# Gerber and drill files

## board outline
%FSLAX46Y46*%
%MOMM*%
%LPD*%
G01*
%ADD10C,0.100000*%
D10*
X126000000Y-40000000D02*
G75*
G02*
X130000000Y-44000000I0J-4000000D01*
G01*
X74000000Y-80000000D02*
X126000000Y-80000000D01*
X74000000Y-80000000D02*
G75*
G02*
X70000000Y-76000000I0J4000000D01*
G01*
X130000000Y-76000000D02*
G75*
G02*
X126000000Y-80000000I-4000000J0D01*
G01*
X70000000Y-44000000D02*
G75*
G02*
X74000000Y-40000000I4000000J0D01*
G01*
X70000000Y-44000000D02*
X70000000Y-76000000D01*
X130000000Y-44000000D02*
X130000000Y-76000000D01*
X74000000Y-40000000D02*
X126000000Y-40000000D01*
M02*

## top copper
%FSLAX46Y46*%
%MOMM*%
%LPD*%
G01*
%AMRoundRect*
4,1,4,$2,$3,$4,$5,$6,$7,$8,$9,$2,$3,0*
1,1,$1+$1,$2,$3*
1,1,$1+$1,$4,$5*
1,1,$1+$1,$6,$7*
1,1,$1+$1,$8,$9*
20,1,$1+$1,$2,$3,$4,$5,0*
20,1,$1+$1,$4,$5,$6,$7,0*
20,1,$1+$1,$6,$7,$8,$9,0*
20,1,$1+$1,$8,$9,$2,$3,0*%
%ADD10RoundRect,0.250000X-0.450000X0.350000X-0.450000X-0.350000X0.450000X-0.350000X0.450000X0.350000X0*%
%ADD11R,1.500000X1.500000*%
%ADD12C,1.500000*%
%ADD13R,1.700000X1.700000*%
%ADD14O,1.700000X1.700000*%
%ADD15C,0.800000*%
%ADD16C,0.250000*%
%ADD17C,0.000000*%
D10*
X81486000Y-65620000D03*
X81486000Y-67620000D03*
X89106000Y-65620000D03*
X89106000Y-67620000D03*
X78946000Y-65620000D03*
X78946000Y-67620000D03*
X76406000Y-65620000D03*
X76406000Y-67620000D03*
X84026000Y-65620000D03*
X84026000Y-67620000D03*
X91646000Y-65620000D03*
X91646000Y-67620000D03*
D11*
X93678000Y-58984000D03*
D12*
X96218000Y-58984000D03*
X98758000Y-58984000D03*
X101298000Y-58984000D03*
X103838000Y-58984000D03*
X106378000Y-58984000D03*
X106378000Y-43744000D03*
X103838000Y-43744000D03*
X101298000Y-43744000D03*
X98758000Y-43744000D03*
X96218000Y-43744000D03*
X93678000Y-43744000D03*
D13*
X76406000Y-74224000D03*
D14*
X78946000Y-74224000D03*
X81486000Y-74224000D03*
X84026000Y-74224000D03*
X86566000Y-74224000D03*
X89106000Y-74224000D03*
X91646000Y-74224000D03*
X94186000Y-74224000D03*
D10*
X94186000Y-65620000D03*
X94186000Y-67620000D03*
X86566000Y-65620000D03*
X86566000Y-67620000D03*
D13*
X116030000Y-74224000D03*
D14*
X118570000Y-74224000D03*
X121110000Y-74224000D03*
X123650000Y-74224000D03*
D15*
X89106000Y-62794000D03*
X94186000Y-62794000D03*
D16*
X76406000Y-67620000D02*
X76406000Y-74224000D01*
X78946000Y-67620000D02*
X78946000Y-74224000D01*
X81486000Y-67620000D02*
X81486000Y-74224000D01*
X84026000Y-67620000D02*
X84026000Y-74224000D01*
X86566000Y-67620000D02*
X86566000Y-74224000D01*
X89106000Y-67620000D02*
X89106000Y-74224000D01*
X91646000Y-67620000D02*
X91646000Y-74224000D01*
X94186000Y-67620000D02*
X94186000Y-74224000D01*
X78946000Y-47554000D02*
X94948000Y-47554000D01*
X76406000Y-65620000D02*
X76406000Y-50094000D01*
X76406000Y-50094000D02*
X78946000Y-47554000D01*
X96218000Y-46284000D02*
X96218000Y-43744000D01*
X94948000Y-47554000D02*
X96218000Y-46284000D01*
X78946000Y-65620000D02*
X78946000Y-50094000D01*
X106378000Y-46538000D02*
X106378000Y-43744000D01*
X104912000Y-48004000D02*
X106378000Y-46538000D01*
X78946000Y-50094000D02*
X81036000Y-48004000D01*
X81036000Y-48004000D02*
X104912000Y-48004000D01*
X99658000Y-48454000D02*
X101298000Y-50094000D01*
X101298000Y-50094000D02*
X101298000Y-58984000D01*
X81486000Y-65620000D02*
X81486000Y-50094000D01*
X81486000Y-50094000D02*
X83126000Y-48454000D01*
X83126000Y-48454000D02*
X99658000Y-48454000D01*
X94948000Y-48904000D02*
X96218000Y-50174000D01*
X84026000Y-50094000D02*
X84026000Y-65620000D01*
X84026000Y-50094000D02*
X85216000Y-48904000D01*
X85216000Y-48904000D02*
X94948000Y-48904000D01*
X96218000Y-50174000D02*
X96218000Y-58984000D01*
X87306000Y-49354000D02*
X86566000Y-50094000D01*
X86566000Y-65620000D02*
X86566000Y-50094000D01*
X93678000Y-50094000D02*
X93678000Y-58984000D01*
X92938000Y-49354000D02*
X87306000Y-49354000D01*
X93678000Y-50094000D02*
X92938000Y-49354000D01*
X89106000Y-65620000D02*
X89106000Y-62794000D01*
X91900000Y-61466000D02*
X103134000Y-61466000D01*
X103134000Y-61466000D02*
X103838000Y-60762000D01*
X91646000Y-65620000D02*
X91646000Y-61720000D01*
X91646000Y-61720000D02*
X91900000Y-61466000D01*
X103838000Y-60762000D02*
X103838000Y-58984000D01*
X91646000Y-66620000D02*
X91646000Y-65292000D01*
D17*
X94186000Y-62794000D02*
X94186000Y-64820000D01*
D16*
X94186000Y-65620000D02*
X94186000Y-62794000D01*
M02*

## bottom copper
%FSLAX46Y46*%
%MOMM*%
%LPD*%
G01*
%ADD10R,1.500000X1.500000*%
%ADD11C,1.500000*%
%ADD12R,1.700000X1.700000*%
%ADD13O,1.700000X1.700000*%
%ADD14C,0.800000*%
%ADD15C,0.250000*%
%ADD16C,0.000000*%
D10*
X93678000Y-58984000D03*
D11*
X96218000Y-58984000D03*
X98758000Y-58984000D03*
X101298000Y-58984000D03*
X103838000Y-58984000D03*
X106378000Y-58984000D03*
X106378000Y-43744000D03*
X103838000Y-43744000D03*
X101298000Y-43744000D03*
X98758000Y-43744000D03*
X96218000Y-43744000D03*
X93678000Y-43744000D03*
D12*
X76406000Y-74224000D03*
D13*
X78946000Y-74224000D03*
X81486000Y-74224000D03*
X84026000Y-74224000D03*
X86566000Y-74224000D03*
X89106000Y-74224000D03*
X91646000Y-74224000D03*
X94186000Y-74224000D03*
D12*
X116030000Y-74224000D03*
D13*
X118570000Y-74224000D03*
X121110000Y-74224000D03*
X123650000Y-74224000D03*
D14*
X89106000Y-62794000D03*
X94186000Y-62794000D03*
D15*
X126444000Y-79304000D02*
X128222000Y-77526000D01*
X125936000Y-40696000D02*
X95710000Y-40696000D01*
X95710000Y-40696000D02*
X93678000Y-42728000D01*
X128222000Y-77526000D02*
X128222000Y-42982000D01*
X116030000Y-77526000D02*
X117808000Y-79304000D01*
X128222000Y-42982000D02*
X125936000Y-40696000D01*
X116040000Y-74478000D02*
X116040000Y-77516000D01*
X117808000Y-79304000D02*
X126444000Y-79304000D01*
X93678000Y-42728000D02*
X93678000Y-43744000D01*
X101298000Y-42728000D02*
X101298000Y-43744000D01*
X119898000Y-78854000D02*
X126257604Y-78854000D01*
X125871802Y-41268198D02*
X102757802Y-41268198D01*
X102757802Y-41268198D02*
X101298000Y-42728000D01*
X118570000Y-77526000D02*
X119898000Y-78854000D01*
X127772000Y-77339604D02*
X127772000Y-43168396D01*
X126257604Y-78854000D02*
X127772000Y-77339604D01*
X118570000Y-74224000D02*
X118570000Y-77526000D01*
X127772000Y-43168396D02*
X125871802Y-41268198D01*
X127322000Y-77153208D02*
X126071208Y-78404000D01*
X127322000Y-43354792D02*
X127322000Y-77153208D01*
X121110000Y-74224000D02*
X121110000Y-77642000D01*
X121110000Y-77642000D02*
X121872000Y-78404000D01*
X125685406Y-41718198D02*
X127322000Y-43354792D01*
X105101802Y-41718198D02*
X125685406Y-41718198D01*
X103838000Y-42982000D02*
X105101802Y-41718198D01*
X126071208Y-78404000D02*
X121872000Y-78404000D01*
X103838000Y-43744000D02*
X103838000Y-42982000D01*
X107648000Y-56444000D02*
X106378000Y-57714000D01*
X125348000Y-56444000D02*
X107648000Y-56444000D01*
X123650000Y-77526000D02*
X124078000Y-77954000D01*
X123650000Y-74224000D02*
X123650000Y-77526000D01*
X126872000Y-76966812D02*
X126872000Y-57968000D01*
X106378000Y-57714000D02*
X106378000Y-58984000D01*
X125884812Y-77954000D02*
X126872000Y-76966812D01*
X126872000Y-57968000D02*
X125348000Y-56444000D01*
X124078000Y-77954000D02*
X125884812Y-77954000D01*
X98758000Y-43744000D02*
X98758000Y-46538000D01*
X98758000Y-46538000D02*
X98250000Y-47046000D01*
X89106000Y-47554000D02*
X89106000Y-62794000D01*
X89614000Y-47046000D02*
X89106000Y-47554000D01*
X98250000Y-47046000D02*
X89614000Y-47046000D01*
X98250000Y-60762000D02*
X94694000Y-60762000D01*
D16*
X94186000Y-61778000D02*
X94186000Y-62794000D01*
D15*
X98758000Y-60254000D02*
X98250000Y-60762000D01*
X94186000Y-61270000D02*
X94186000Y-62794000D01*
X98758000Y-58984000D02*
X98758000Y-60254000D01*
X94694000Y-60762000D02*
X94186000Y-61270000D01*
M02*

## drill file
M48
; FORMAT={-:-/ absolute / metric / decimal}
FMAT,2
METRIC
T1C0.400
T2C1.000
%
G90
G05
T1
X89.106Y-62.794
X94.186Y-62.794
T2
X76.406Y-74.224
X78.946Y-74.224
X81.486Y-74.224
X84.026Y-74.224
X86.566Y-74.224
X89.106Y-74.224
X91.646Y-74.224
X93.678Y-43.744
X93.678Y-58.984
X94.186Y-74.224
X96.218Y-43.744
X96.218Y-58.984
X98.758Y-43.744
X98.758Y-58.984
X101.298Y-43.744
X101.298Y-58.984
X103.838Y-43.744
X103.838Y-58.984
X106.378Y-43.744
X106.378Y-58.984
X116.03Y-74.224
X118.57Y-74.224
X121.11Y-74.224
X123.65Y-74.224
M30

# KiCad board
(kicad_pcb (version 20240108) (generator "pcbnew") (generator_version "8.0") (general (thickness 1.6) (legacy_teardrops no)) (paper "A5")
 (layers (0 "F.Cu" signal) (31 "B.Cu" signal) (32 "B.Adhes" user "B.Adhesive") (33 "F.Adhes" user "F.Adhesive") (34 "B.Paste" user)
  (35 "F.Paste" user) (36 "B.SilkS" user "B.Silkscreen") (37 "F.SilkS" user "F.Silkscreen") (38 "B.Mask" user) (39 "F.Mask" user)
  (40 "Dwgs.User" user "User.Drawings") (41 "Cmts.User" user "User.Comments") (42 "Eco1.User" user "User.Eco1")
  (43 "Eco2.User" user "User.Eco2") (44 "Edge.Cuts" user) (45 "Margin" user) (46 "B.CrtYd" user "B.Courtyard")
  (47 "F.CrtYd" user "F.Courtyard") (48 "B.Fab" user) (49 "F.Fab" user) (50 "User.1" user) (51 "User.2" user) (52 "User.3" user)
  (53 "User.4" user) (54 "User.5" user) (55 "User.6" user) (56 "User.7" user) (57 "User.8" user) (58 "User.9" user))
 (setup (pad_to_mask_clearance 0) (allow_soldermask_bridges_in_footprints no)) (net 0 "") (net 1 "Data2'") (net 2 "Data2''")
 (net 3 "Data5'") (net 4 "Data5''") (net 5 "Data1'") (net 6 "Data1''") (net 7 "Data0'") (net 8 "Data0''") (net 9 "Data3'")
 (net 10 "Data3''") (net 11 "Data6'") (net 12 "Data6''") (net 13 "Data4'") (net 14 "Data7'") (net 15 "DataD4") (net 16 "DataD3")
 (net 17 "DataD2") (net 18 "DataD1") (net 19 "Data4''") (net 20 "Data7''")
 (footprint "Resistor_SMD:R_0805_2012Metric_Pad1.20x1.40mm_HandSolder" (layer "F.Cu") (at 81.486 66.62 -90)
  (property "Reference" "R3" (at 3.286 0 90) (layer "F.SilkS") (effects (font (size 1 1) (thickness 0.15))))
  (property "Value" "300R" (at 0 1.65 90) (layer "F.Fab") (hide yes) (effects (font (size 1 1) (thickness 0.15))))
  (pad "1" smd roundrect (at -1 0 270) (size 1.2 1.4) (layers "F.Cu" "F.Paste" "F.Mask") (roundrect_rratio 0.2083333333) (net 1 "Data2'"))
  (pad "2" smd roundrect (at 1 0 270) (size 1.2 1.4) (layers "F.Cu" "F.Paste" "F.Mask") (roundrect_rratio 0.2083333333) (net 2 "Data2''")))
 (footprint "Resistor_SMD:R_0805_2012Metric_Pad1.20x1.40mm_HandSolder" (layer "F.Cu") (at 89.106 66.62 -90)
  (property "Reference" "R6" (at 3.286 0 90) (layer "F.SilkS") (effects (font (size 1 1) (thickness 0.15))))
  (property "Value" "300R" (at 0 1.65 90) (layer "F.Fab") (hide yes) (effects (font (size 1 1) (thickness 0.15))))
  (pad "1" smd roundrect (at -1 0 270) (size 1.2 1.4) (layers "F.Cu" "F.Paste" "F.Mask") (roundrect_rratio 0.2083333333) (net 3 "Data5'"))
  (pad "2" smd roundrect (at 1 0 270) (size 1.2 1.4) (layers "F.Cu" "F.Paste" "F.Mask") (roundrect_rratio 0.2083333333) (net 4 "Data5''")))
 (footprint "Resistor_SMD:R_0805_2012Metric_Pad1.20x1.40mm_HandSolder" (layer "F.Cu") (at 78.946 66.62 -90)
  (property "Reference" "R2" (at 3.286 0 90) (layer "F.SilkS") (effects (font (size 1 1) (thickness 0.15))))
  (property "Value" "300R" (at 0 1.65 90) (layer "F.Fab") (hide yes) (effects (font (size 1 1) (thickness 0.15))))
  (pad "1" smd roundrect (at -1 0 270) (size 1.2 1.4) (layers "F.Cu" "F.Paste" "F.Mask") (roundrect_rratio 0.2083333333) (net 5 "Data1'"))
  (pad "2" smd roundrect (at 1 0 270) (size 1.2 1.4) (layers "F.Cu" "F.Paste" "F.Mask") (roundrect_rratio 0.2083333333) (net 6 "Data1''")))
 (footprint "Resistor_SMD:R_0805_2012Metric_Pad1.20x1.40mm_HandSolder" (layer "F.Cu") (at 76.406 66.62 -90)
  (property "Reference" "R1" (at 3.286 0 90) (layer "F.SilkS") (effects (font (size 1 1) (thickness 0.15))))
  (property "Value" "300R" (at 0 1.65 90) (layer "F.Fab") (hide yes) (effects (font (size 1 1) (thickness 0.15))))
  (pad "1" smd roundrect (at -1 0 270) (size 1.2 1.4) (layers "F.Cu" "F.Paste" "F.Mask") (roundrect_rratio 0.2083333333) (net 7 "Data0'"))
  (pad "2" smd roundrect (at 1 0 270) (size 1.2 1.4) (layers "F.Cu" "F.Paste" "F.Mask") (roundrect_rratio 0.2083333333) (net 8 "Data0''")))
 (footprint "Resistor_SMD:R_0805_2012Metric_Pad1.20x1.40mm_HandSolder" (layer "F.Cu") (at 84.026 66.62 -90)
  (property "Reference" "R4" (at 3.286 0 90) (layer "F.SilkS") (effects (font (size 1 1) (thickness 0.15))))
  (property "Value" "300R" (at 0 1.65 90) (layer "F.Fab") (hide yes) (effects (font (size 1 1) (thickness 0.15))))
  (pad "1" smd roundrect (at -1 0 270) (size 1.2 1.4) (layers "F.Cu" "F.Paste" "F.Mask") (roundrect_rratio 0.2083333333) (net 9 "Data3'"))
  (pad "2" smd roundrect (at 1 0 270) (size 1.2 1.4) (layers "F.Cu" "F.Paste" "F.Mask") (roundrect_rratio 0.2083333333) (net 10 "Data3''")))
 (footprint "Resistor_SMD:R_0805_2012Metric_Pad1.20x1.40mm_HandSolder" (layer "F.Cu") (at 91.646 66.62 -90)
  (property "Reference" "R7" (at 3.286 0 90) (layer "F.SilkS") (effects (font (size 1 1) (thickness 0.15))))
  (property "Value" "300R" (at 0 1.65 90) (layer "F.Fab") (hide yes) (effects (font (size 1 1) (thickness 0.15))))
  (pad "1" smd roundrect (at -1 0 270) (size 1.2 1.4) (layers "F.Cu" "F.Paste" "F.Mask") (roundrect_rratio 0.2083333333) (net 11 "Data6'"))
  (pad "2" smd roundrect (at 1 0 270) (size 1.2 1.4) (layers "F.Cu" "F.Paste" "F.Mask") (roundrect_rratio 0.2083333333) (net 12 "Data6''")))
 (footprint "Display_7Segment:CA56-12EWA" (layer "F.Cu") (at 93.678 58.984 90)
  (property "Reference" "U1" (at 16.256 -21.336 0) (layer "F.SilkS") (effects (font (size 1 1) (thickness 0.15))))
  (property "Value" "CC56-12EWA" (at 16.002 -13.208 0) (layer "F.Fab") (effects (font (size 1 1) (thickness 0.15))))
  (pad "1" thru_hole rect (at 0 0 90) (size 1.5 1.5) (drill 1) (layers "*.Cu" "*.Mask") (remove_unused_layers no) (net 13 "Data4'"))
  (pad "2" thru_hole circle (at 0 2.54 90) (size 1.5 1.5) (drill 1) (layers "*.Cu" "*.Mask") (remove_unused_layers no) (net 9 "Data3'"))
  (pad "3" thru_hole circle (at 0 5.08 90) (size 1.5 1.5) (drill 1) (layers "*.Cu" "*.Mask") (remove_unused_layers no) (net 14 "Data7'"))
  (pad "4" thru_hole circle (at 0 7.62 90) (size 1.5 1.5) (drill 1) (layers "*.Cu" "*.Mask") (remove_unused_layers no) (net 1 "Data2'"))
  (pad "5" thru_hole circle (at 0 10.16 90) (size 1.5 1.5) (drill 1) (layers "*.Cu" "*.Mask") (remove_unused_layers no) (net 11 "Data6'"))
  (pad "6" thru_hole circle (at 0 12.7 90) (size 1.5 1.5) (drill 1) (layers "*.Cu" "*.Mask") (remove_unused_layers no) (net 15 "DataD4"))
  (pad "7" thru_hole circle (at 15.24 12.7 90) (size 1.5 1.5) (drill 1) (layers "*.Cu" "*.Mask") (remove_unused_layers no) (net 5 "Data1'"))
  (pad "8" thru_hole circle (at 15.24 10.16 90) (size 1.5 1.5) (drill 1) (layers "*.Cu" "*.Mask") (remove_unused_layers no)
   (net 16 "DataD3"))
  (pad "9" thru_hole circle (at 15.24 7.62 90) (size 1.5 1.5) (drill 1) (layers "*.Cu" "*.Mask") (remove_unused_layers no) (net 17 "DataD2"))
  (pad "10" thru_hole circle (at 15.24 5.08 90) (size 1.5 1.5) (drill 1) (layers "*.Cu" "*.Mask") (remove_unused_layers no) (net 3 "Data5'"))
  (pad "11" thru_hole circle (at 15.24 2.54 90) (size 1.5 1.5) (drill 1) (layers "*.Cu" "*.Mask") (remove_unused_layers no) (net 7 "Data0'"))
  (pad "12" thru_hole circle (at 15.24 0 90) (size 1.5 1.5) (drill 1) (layers "*.Cu" "*.Mask") (remove_unused_layers no) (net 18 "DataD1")))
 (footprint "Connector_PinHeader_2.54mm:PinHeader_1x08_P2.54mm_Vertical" (layer "F.Cu") (at 76.406 74.224 90)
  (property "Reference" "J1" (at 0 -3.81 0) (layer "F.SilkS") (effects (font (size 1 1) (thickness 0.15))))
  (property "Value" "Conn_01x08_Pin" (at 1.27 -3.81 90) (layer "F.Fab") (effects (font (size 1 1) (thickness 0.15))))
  (pad "1" thru_hole rect (at 0 0 90) (size 1.7 1.7) (drill 1) (layers "*.Cu" "*.Mask") (remove_unused_layers no) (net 8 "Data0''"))
  (pad "2" thru_hole oval (at 0 2.54 90) (size 1.7 1.7) (drill 1) (layers "*.Cu" "*.Mask") (remove_unused_layers no) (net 6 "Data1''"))
  (pad "3" thru_hole oval (at 0 5.08 90) (size 1.7 1.7) (drill 1) (layers "*.Cu" "*.Mask") (remove_unused_layers no) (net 2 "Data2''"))
  (pad "4" thru_hole oval (at 0 7.62 90) (size 1.7 1.7) (drill 1) (layers "*.Cu" "*.Mask") (remove_unused_layers no) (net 10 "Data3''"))
  (pad "5" thru_hole oval (at 0 10.16 90) (size 1.7 1.7) (drill 1) (layers "*.Cu" "*.Mask") (remove_unused_layers no) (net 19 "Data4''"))
  (pad "6" thru_hole oval (at 0 12.7 90) (size 1.7 1.7) (drill 1) (layers "*.Cu" "*.Mask") (remove_unused_layers no) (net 4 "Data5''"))
  (pad "7" thru_hole oval (at 0 15.24 90) (size 1.7 1.7) (drill 1) (layers "*.Cu" "*.Mask") (remove_unused_layers no) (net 12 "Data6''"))
  (pad "8" thru_hole oval (at 0 17.78 90) (size 1.7 1.7) (drill 1) (layers "*.Cu" "*.Mask") (remove_unused_layers no) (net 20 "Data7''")))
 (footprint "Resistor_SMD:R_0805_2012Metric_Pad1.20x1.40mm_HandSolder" (layer "F.Cu") (at 94.186 66.62 -90)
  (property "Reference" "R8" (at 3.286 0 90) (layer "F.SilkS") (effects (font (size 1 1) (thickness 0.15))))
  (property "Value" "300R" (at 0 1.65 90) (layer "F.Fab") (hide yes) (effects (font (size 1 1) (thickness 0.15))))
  (pad "1" smd roundrect (at -1 0 270) (size 1.2 1.4) (layers "F.Cu" "F.Paste" "F.Mask") (roundrect_rratio 0.2083333333) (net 14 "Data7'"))
  (pad "2" smd roundrect (at 1 0 270) (size 1.2 1.4) (layers "F.Cu" "F.Paste" "F.Mask") (roundrect_rratio 0.2083333333) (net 20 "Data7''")))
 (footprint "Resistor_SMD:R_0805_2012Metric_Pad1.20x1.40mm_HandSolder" (layer "F.Cu") (at 86.566 66.62 -90)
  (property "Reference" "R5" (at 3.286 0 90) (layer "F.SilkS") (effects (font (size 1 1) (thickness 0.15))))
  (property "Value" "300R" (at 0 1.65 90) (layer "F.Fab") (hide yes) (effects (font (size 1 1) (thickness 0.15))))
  (pad "1" smd roundrect (at -1 0 270) (size 1.2 1.4) (layers "F.Cu" "F.Paste" "F.Mask") (roundrect_rratio 0.2083333333) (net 13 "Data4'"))
  (pad "2" smd roundrect (at 1 0 270) (size 1.2 1.4) (layers "F.Cu" "F.Paste" "F.Mask") (roundrect_rratio 0.2083333333) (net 19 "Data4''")))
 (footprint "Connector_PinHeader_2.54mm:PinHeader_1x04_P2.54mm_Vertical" (layer "F.Cu") (at 116.03 74.224 90)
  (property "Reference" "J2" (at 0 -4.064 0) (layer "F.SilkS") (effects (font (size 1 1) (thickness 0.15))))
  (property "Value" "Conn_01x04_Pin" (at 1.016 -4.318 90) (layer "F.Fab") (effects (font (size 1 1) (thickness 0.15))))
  (pad "1" thru_hole rect (at 0 0 90) (size 1.7 1.7) (drill 1) (layers "*.Cu" "*.Mask") (remove_unused_layers no) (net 18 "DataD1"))
  (pad "2" thru_hole oval (at 0 2.54 90) (size 1.7 1.7) (drill 1) (layers "*.Cu" "*.Mask") (remove_unused_layers no) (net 17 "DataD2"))
  (pad "3" thru_hole oval (at 0 5.08 90) (size 1.7 1.7) (drill 1) (layers "*.Cu" "*.Mask") (remove_unused_layers no) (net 16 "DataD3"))
  (pad "4" thru_hole oval (at 0 7.62 90) (size 1.7 1.7) (drill 1) (layers "*.Cu" "*.Mask") (remove_unused_layers no) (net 15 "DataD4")))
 (gr_arc (start 126 40) (mid 128.828427 41.171573) (end 130 44) (stroke (width 0.1) (type default)) (layer "Edge.Cuts"))
 (gr_line (start 74 80) (end 126 80) (stroke (width 0.1) (type default)) (layer "Edge.Cuts"))
 (gr_arc (start 74 80) (mid 71.171573 78.828427) (end 70 76) (stroke (width 0.1) (type default)) (layer "Edge.Cuts"))
 (gr_arc (start 130 76) (mid 128.828427 78.828427) (end 126 80) (stroke (width 0.1) (type default)) (layer "Edge.Cuts"))
 (gr_arc (start 70 44) (mid 71.171573 41.171573) (end 74 40) (stroke (width 0.1) (type default)) (layer "Edge.Cuts"))
 (gr_line (start 70 44) (end 70 76) (stroke (width 0.1) (type default)) (layer "Edge.Cuts"))
 (gr_line (start 130 44) (end 130 76) (stroke (width 0.1) (type default)) (layer "Edge.Cuts"))
 (gr_line (start 74 40) (end 126 40) (stroke (width 0.1) (type default)) (layer "Edge.Cuts"))
 (segment (start 76.406 67.62) (end 76.406 74.224) (width 0.25) (layer "F.Cu") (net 8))
 (segment (start 78.946 67.62) (end 78.946 74.224) (width 0.25) (layer "F.Cu") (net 6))
 (segment (start 81.486 67.62) (end 81.486 74.224) (width 0.25) (layer "F.Cu") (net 2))
 (segment (start 84.026 67.62) (end 84.026 74.224) (width 0.25) (layer "F.Cu") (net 10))
 (segment (start 86.566 67.62) (end 86.566 74.224) (width 0.25) (layer "F.Cu") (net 19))
 (segment (start 89.106 67.62) (end 89.106 74.224) (width 0.25) (layer "F.Cu") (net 4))
 (segment (start 91.646 67.62) (end 91.646 74.224) (width 0.25) (layer "F.Cu") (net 12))
 (segment (start 94.186 67.62) (end 94.186 74.224) (width 0.25) (layer "F.Cu") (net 20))
 (segment (start 126.444 79.304) (end 128.222 77.526) (width 0.25) (layer "B.Cu") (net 18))
 (segment (start 125.936 40.696) (end 95.71 40.696) (width 0.25) (layer "B.Cu") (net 18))
 (segment (start 95.71 40.696) (end 93.678 42.728) (width 0.25) (layer "B.Cu") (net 18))
 (segment (start 128.222 77.526) (end 128.222 42.982) (width 0.25) (layer "B.Cu") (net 18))
 (segment (start 116.03 77.526) (end 117.808 79.304) (width 0.25) (layer "B.Cu") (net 18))
 (segment (start 128.222 42.982) (end 125.936 40.696) (width 0.25) (layer "B.Cu") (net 18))
 (segment (start 116.04 74.478) (end 116.04 77.516) (width 0.25) (layer "B.Cu") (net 18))
 (segment (start 117.808 79.304) (end 126.444 79.304) (width 0.25) (layer "B.Cu") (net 18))
 (segment (start 93.678 42.728) (end 93.678 43.744) (width 0.25) (layer "B.Cu") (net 18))
 (segment (start 101.298 42.728) (end 101.298 43.744) (width 0.25) (layer "B.Cu") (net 17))
 (segment (start 119.898 78.854) (end 126.257604 78.854) (width 0.25) (layer "B.Cu") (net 17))
 (segment (start 125.871802 41.268198) (end 102.757802 41.268198) (width 0.25) (layer "B.Cu") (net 17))
 (segment (start 102.757802 41.268198) (end 101.298 42.728) (width 0.25) (layer "B.Cu") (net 17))
 (segment (start 118.57 77.526) (end 119.898 78.854) (width 0.25) (layer "B.Cu") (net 17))
 (segment (start 127.772 77.339604) (end 127.772 43.168396) (width 0.25) (layer "B.Cu") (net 17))
 (segment (start 126.257604 78.854) (end 127.772 77.339604) (width 0.25) (layer "B.Cu") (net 17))
 (segment (start 118.57 74.224) (end 118.57 77.526) (width 0.25) (layer "B.Cu") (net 17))
 (segment (start 127.772 43.168396) (end 125.871802 41.268198) (width 0.25) (layer "B.Cu") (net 17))
 (segment (start 127.322 77.153208) (end 126.071208 78.404) (width 0.25) (layer "B.Cu") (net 16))
 (segment (start 127.322 43.354792) (end 127.322 77.153208) (width 0.25) (layer "B.Cu") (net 16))
 (segment (start 121.11 74.224) (end 121.11 77.642) (width 0.25) (layer "B.Cu") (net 16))
 (segment (start 121.11 77.642) (end 121.872 78.404) (width 0.25) (layer "B.Cu") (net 16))
 (segment (start 125.685406 41.718198) (end 127.322 43.354792) (width 0.25) (layer "B.Cu") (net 16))
 (segment (start 105.101802 41.718198) (end 125.685406 41.718198) (width 0.25) (layer "B.Cu") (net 16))
 (segment (start 103.838 42.982) (end 105.101802 41.718198) (width 0.25) (layer "B.Cu") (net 16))
 (segment (start 126.071208 78.404) (end 121.872 78.404) (width 0.25) (layer "B.Cu") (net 16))
 (segment (start 103.838 43.744) (end 103.838 42.982) (width 0.25) (layer "B.Cu") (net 16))
 (segment (start 107.648 56.444) (end 106.378 57.714) (width 0.25) (layer "B.Cu") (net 15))
 (segment (start 125.348 56.444) (end 107.648 56.444) (width 0.25) (layer "B.Cu") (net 15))
 (segment (start 123.65 77.526) (end 124.078 77.954) (width 0.25) (layer "B.Cu") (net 15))
 (segment (start 123.65 74.224) (end 123.65 77.526) (width 0.25) (layer "B.Cu") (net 15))
 (segment (start 126.872 76.966812) (end 126.872 57.968) (width 0.25) (layer "B.Cu") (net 15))
 (segment (start 106.378 57.714) (end 106.378 58.984) (width 0.25) (layer "B.Cu") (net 15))
 (segment (start 125.884812 77.954) (end 126.872 76.966812) (width 0.25) (layer "B.Cu") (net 15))
 (segment (start 126.872 57.968) (end 125.348 56.444) (width 0.25) (layer "B.Cu") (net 15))
 (segment (start 124.078 77.954) (end 125.884812 77.954) (width 0.25) (layer "B.Cu") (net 15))
 (segment (start 78.946 47.554) (end 94.948 47.554) (width 0.25) (layer "F.Cu") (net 7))
 (segment (start 76.406 65.62) (end 76.406 50.094) (width 0.25) (layer "F.Cu") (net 7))
 (segment (start 76.406 50.094) (end 78.946 47.554) (width 0.25) (layer "F.Cu") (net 7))
 (segment (start 96.218 46.284) (end 96.218 43.744) (width 0.25) (layer "F.Cu") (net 7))
 (segment (start 94.948 47.554) (end 96.218 46.284) (width 0.25) (layer "F.Cu") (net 7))
 (segment (start 78.946 65.62) (end 78.946 50.094) (width 0.25) (layer "F.Cu") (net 5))
 (segment (start 106.378 46.538) (end 106.378 43.744) (width 0.25) (layer "F.Cu") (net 5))
 (segment (start 104.912 48.004) (end 106.378 46.538) (width 0.25) (layer "F.Cu") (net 5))
 (segment (start 78.946 50.094) (end 81.036 48.004) (width 0.25) (layer "F.Cu") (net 5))
 (segment (start 81.036 48.004) (end 104.912 48.004) (width 0.25) (layer "F.Cu") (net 5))
 (segment (start 99.658 48.454) (end 101.298 50.094) (width 0.25) (layer "F.Cu") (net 1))
 (segment (start 101.298 50.094) (end 101.298 58.984) (width 0.25) (layer "F.Cu") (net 1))
 (segment (start 81.486 65.62) (end 81.486 50.094) (width 0.25) (layer "F.Cu") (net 1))
 (segment (start 81.486 50.094) (end 83.126 48.454) (width 0.25) (layer "F.Cu") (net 1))
 (segment (start 83.126 48.454) (end 99.658 48.454) (width 0.25) (layer "F.Cu") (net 1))
 (segment (start 94.948 48.904) (end 96.218 50.174) (width 0.25) (layer "F.Cu") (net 9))
 (segment (start 84.026 50.094) (end 84.026 65.62) (width 0.25) (layer "F.Cu") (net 9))
 (segment (start 84.026 50.094) (end 85.216 48.904) (width 0.25) (layer "F.Cu") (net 9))
 (segment (start 85.216 48.904) (end 94.948 48.904) (width 0.25) (layer "F.Cu") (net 9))
 (segment (start 96.218 50.174) (end 96.218 58.984) (width 0.25) (layer "F.Cu") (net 9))
 (segment (start 87.306 49.354) (end 86.566 50.094) (width 0.25) (layer "F.Cu") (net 13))
 (segment (start 86.566 65.62) (end 86.566 50.094) (width 0.25) (layer "F.Cu") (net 13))
 (segment (start 93.678 50.094) (end 93.678 58.984) (width 0.25) (layer "F.Cu") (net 13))
 (segment (start 92.938 49.354) (end 87.306 49.354) (width 0.25) (layer "F.Cu") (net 13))
 (segment (start 93.678 50.094) (end 92.938 49.354) (width 0.25) (layer "F.Cu") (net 13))
 (segment (start 89.106 65.62) (end 89.106 62.794) (width 0.25) (layer "F.Cu") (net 3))
 (via (at 89.106 62.794) (size 0.8) (drill 0.4) (layers "F.Cu" "B.Cu") (free yes) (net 3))
 (segment (start 98.758 43.744) (end 98.758 46.538) (width 0.25) (layer "B.Cu") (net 3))
 (segment (start 98.758 46.538) (end 98.25 47.046) (width 0.25) (layer "B.Cu") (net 3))
 (segment (start 89.106 47.554) (end 89.106 62.794) (width 0.25) (layer "B.Cu") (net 3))
 (segment (start 89.614 47.046) (end 89.106 47.554) (width 0.25) (layer "B.Cu") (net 3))
 (segment (start 98.25 47.046) (end 89.614 47.046) (width 0.25) (layer "B.Cu") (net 3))
 (segment (start 91.9 61.466) (end 103.134 61.466) (width 0.25) (layer "F.Cu") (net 11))
 (segment (start 103.134 61.466) (end 103.838 60.762) (width 0.25) (layer "F.Cu") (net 11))
 (segment (start 91.646 65.62) (end 91.646 61.72) (width 0.25) (layer "F.Cu") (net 11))
 (segment (start 91.646 61.72) (end 91.9 61.466) (width 0.25) (layer "F.Cu") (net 11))
 (segment (start 103.838 60.762) (end 103.838 58.984) (width 0.25) (layer "F.Cu") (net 11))
 (segment (start 91.646 66.62) (end 91.646 65.292) (width 0.25) (layer "F.Cu") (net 11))
 (segment (start 94.186 62.794) (end 94.186 64.82) (width 0) (layer "F.Cu") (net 14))
 (segment (start 94.186 65.62) (end 94.186 62.794) (width 0.25) (layer "F.Cu") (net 14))
 (via (at 94.186 62.794) (size 0.8) (drill 0.4) (layers "F.Cu" "B.Cu") (free yes) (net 14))
 (segment (start 98.25 60.762) (end 94.694 60.762) (width 0.25) (layer "B.Cu") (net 14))
 (segment (start 94.186 61.778) (end 94.186 62.794) (width 0) (layer "B.Cu") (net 14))
 (segment (start 98.758 60.254) (end 98.25 60.762) (width 0.25) (layer "B.Cu") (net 14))
 (segment (start 94.186 61.27) (end 94.186 62.794) (width 0.25) (layer "B.Cu") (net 14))
 (segment (start 98.758 58.984) (end 98.758 60.254) (width 0.25) (layer "B.Cu") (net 14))
 (segment (start 94.694 60.762) (end 94.186 61.27) (width 0.25) (layer "B.Cu") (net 14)))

